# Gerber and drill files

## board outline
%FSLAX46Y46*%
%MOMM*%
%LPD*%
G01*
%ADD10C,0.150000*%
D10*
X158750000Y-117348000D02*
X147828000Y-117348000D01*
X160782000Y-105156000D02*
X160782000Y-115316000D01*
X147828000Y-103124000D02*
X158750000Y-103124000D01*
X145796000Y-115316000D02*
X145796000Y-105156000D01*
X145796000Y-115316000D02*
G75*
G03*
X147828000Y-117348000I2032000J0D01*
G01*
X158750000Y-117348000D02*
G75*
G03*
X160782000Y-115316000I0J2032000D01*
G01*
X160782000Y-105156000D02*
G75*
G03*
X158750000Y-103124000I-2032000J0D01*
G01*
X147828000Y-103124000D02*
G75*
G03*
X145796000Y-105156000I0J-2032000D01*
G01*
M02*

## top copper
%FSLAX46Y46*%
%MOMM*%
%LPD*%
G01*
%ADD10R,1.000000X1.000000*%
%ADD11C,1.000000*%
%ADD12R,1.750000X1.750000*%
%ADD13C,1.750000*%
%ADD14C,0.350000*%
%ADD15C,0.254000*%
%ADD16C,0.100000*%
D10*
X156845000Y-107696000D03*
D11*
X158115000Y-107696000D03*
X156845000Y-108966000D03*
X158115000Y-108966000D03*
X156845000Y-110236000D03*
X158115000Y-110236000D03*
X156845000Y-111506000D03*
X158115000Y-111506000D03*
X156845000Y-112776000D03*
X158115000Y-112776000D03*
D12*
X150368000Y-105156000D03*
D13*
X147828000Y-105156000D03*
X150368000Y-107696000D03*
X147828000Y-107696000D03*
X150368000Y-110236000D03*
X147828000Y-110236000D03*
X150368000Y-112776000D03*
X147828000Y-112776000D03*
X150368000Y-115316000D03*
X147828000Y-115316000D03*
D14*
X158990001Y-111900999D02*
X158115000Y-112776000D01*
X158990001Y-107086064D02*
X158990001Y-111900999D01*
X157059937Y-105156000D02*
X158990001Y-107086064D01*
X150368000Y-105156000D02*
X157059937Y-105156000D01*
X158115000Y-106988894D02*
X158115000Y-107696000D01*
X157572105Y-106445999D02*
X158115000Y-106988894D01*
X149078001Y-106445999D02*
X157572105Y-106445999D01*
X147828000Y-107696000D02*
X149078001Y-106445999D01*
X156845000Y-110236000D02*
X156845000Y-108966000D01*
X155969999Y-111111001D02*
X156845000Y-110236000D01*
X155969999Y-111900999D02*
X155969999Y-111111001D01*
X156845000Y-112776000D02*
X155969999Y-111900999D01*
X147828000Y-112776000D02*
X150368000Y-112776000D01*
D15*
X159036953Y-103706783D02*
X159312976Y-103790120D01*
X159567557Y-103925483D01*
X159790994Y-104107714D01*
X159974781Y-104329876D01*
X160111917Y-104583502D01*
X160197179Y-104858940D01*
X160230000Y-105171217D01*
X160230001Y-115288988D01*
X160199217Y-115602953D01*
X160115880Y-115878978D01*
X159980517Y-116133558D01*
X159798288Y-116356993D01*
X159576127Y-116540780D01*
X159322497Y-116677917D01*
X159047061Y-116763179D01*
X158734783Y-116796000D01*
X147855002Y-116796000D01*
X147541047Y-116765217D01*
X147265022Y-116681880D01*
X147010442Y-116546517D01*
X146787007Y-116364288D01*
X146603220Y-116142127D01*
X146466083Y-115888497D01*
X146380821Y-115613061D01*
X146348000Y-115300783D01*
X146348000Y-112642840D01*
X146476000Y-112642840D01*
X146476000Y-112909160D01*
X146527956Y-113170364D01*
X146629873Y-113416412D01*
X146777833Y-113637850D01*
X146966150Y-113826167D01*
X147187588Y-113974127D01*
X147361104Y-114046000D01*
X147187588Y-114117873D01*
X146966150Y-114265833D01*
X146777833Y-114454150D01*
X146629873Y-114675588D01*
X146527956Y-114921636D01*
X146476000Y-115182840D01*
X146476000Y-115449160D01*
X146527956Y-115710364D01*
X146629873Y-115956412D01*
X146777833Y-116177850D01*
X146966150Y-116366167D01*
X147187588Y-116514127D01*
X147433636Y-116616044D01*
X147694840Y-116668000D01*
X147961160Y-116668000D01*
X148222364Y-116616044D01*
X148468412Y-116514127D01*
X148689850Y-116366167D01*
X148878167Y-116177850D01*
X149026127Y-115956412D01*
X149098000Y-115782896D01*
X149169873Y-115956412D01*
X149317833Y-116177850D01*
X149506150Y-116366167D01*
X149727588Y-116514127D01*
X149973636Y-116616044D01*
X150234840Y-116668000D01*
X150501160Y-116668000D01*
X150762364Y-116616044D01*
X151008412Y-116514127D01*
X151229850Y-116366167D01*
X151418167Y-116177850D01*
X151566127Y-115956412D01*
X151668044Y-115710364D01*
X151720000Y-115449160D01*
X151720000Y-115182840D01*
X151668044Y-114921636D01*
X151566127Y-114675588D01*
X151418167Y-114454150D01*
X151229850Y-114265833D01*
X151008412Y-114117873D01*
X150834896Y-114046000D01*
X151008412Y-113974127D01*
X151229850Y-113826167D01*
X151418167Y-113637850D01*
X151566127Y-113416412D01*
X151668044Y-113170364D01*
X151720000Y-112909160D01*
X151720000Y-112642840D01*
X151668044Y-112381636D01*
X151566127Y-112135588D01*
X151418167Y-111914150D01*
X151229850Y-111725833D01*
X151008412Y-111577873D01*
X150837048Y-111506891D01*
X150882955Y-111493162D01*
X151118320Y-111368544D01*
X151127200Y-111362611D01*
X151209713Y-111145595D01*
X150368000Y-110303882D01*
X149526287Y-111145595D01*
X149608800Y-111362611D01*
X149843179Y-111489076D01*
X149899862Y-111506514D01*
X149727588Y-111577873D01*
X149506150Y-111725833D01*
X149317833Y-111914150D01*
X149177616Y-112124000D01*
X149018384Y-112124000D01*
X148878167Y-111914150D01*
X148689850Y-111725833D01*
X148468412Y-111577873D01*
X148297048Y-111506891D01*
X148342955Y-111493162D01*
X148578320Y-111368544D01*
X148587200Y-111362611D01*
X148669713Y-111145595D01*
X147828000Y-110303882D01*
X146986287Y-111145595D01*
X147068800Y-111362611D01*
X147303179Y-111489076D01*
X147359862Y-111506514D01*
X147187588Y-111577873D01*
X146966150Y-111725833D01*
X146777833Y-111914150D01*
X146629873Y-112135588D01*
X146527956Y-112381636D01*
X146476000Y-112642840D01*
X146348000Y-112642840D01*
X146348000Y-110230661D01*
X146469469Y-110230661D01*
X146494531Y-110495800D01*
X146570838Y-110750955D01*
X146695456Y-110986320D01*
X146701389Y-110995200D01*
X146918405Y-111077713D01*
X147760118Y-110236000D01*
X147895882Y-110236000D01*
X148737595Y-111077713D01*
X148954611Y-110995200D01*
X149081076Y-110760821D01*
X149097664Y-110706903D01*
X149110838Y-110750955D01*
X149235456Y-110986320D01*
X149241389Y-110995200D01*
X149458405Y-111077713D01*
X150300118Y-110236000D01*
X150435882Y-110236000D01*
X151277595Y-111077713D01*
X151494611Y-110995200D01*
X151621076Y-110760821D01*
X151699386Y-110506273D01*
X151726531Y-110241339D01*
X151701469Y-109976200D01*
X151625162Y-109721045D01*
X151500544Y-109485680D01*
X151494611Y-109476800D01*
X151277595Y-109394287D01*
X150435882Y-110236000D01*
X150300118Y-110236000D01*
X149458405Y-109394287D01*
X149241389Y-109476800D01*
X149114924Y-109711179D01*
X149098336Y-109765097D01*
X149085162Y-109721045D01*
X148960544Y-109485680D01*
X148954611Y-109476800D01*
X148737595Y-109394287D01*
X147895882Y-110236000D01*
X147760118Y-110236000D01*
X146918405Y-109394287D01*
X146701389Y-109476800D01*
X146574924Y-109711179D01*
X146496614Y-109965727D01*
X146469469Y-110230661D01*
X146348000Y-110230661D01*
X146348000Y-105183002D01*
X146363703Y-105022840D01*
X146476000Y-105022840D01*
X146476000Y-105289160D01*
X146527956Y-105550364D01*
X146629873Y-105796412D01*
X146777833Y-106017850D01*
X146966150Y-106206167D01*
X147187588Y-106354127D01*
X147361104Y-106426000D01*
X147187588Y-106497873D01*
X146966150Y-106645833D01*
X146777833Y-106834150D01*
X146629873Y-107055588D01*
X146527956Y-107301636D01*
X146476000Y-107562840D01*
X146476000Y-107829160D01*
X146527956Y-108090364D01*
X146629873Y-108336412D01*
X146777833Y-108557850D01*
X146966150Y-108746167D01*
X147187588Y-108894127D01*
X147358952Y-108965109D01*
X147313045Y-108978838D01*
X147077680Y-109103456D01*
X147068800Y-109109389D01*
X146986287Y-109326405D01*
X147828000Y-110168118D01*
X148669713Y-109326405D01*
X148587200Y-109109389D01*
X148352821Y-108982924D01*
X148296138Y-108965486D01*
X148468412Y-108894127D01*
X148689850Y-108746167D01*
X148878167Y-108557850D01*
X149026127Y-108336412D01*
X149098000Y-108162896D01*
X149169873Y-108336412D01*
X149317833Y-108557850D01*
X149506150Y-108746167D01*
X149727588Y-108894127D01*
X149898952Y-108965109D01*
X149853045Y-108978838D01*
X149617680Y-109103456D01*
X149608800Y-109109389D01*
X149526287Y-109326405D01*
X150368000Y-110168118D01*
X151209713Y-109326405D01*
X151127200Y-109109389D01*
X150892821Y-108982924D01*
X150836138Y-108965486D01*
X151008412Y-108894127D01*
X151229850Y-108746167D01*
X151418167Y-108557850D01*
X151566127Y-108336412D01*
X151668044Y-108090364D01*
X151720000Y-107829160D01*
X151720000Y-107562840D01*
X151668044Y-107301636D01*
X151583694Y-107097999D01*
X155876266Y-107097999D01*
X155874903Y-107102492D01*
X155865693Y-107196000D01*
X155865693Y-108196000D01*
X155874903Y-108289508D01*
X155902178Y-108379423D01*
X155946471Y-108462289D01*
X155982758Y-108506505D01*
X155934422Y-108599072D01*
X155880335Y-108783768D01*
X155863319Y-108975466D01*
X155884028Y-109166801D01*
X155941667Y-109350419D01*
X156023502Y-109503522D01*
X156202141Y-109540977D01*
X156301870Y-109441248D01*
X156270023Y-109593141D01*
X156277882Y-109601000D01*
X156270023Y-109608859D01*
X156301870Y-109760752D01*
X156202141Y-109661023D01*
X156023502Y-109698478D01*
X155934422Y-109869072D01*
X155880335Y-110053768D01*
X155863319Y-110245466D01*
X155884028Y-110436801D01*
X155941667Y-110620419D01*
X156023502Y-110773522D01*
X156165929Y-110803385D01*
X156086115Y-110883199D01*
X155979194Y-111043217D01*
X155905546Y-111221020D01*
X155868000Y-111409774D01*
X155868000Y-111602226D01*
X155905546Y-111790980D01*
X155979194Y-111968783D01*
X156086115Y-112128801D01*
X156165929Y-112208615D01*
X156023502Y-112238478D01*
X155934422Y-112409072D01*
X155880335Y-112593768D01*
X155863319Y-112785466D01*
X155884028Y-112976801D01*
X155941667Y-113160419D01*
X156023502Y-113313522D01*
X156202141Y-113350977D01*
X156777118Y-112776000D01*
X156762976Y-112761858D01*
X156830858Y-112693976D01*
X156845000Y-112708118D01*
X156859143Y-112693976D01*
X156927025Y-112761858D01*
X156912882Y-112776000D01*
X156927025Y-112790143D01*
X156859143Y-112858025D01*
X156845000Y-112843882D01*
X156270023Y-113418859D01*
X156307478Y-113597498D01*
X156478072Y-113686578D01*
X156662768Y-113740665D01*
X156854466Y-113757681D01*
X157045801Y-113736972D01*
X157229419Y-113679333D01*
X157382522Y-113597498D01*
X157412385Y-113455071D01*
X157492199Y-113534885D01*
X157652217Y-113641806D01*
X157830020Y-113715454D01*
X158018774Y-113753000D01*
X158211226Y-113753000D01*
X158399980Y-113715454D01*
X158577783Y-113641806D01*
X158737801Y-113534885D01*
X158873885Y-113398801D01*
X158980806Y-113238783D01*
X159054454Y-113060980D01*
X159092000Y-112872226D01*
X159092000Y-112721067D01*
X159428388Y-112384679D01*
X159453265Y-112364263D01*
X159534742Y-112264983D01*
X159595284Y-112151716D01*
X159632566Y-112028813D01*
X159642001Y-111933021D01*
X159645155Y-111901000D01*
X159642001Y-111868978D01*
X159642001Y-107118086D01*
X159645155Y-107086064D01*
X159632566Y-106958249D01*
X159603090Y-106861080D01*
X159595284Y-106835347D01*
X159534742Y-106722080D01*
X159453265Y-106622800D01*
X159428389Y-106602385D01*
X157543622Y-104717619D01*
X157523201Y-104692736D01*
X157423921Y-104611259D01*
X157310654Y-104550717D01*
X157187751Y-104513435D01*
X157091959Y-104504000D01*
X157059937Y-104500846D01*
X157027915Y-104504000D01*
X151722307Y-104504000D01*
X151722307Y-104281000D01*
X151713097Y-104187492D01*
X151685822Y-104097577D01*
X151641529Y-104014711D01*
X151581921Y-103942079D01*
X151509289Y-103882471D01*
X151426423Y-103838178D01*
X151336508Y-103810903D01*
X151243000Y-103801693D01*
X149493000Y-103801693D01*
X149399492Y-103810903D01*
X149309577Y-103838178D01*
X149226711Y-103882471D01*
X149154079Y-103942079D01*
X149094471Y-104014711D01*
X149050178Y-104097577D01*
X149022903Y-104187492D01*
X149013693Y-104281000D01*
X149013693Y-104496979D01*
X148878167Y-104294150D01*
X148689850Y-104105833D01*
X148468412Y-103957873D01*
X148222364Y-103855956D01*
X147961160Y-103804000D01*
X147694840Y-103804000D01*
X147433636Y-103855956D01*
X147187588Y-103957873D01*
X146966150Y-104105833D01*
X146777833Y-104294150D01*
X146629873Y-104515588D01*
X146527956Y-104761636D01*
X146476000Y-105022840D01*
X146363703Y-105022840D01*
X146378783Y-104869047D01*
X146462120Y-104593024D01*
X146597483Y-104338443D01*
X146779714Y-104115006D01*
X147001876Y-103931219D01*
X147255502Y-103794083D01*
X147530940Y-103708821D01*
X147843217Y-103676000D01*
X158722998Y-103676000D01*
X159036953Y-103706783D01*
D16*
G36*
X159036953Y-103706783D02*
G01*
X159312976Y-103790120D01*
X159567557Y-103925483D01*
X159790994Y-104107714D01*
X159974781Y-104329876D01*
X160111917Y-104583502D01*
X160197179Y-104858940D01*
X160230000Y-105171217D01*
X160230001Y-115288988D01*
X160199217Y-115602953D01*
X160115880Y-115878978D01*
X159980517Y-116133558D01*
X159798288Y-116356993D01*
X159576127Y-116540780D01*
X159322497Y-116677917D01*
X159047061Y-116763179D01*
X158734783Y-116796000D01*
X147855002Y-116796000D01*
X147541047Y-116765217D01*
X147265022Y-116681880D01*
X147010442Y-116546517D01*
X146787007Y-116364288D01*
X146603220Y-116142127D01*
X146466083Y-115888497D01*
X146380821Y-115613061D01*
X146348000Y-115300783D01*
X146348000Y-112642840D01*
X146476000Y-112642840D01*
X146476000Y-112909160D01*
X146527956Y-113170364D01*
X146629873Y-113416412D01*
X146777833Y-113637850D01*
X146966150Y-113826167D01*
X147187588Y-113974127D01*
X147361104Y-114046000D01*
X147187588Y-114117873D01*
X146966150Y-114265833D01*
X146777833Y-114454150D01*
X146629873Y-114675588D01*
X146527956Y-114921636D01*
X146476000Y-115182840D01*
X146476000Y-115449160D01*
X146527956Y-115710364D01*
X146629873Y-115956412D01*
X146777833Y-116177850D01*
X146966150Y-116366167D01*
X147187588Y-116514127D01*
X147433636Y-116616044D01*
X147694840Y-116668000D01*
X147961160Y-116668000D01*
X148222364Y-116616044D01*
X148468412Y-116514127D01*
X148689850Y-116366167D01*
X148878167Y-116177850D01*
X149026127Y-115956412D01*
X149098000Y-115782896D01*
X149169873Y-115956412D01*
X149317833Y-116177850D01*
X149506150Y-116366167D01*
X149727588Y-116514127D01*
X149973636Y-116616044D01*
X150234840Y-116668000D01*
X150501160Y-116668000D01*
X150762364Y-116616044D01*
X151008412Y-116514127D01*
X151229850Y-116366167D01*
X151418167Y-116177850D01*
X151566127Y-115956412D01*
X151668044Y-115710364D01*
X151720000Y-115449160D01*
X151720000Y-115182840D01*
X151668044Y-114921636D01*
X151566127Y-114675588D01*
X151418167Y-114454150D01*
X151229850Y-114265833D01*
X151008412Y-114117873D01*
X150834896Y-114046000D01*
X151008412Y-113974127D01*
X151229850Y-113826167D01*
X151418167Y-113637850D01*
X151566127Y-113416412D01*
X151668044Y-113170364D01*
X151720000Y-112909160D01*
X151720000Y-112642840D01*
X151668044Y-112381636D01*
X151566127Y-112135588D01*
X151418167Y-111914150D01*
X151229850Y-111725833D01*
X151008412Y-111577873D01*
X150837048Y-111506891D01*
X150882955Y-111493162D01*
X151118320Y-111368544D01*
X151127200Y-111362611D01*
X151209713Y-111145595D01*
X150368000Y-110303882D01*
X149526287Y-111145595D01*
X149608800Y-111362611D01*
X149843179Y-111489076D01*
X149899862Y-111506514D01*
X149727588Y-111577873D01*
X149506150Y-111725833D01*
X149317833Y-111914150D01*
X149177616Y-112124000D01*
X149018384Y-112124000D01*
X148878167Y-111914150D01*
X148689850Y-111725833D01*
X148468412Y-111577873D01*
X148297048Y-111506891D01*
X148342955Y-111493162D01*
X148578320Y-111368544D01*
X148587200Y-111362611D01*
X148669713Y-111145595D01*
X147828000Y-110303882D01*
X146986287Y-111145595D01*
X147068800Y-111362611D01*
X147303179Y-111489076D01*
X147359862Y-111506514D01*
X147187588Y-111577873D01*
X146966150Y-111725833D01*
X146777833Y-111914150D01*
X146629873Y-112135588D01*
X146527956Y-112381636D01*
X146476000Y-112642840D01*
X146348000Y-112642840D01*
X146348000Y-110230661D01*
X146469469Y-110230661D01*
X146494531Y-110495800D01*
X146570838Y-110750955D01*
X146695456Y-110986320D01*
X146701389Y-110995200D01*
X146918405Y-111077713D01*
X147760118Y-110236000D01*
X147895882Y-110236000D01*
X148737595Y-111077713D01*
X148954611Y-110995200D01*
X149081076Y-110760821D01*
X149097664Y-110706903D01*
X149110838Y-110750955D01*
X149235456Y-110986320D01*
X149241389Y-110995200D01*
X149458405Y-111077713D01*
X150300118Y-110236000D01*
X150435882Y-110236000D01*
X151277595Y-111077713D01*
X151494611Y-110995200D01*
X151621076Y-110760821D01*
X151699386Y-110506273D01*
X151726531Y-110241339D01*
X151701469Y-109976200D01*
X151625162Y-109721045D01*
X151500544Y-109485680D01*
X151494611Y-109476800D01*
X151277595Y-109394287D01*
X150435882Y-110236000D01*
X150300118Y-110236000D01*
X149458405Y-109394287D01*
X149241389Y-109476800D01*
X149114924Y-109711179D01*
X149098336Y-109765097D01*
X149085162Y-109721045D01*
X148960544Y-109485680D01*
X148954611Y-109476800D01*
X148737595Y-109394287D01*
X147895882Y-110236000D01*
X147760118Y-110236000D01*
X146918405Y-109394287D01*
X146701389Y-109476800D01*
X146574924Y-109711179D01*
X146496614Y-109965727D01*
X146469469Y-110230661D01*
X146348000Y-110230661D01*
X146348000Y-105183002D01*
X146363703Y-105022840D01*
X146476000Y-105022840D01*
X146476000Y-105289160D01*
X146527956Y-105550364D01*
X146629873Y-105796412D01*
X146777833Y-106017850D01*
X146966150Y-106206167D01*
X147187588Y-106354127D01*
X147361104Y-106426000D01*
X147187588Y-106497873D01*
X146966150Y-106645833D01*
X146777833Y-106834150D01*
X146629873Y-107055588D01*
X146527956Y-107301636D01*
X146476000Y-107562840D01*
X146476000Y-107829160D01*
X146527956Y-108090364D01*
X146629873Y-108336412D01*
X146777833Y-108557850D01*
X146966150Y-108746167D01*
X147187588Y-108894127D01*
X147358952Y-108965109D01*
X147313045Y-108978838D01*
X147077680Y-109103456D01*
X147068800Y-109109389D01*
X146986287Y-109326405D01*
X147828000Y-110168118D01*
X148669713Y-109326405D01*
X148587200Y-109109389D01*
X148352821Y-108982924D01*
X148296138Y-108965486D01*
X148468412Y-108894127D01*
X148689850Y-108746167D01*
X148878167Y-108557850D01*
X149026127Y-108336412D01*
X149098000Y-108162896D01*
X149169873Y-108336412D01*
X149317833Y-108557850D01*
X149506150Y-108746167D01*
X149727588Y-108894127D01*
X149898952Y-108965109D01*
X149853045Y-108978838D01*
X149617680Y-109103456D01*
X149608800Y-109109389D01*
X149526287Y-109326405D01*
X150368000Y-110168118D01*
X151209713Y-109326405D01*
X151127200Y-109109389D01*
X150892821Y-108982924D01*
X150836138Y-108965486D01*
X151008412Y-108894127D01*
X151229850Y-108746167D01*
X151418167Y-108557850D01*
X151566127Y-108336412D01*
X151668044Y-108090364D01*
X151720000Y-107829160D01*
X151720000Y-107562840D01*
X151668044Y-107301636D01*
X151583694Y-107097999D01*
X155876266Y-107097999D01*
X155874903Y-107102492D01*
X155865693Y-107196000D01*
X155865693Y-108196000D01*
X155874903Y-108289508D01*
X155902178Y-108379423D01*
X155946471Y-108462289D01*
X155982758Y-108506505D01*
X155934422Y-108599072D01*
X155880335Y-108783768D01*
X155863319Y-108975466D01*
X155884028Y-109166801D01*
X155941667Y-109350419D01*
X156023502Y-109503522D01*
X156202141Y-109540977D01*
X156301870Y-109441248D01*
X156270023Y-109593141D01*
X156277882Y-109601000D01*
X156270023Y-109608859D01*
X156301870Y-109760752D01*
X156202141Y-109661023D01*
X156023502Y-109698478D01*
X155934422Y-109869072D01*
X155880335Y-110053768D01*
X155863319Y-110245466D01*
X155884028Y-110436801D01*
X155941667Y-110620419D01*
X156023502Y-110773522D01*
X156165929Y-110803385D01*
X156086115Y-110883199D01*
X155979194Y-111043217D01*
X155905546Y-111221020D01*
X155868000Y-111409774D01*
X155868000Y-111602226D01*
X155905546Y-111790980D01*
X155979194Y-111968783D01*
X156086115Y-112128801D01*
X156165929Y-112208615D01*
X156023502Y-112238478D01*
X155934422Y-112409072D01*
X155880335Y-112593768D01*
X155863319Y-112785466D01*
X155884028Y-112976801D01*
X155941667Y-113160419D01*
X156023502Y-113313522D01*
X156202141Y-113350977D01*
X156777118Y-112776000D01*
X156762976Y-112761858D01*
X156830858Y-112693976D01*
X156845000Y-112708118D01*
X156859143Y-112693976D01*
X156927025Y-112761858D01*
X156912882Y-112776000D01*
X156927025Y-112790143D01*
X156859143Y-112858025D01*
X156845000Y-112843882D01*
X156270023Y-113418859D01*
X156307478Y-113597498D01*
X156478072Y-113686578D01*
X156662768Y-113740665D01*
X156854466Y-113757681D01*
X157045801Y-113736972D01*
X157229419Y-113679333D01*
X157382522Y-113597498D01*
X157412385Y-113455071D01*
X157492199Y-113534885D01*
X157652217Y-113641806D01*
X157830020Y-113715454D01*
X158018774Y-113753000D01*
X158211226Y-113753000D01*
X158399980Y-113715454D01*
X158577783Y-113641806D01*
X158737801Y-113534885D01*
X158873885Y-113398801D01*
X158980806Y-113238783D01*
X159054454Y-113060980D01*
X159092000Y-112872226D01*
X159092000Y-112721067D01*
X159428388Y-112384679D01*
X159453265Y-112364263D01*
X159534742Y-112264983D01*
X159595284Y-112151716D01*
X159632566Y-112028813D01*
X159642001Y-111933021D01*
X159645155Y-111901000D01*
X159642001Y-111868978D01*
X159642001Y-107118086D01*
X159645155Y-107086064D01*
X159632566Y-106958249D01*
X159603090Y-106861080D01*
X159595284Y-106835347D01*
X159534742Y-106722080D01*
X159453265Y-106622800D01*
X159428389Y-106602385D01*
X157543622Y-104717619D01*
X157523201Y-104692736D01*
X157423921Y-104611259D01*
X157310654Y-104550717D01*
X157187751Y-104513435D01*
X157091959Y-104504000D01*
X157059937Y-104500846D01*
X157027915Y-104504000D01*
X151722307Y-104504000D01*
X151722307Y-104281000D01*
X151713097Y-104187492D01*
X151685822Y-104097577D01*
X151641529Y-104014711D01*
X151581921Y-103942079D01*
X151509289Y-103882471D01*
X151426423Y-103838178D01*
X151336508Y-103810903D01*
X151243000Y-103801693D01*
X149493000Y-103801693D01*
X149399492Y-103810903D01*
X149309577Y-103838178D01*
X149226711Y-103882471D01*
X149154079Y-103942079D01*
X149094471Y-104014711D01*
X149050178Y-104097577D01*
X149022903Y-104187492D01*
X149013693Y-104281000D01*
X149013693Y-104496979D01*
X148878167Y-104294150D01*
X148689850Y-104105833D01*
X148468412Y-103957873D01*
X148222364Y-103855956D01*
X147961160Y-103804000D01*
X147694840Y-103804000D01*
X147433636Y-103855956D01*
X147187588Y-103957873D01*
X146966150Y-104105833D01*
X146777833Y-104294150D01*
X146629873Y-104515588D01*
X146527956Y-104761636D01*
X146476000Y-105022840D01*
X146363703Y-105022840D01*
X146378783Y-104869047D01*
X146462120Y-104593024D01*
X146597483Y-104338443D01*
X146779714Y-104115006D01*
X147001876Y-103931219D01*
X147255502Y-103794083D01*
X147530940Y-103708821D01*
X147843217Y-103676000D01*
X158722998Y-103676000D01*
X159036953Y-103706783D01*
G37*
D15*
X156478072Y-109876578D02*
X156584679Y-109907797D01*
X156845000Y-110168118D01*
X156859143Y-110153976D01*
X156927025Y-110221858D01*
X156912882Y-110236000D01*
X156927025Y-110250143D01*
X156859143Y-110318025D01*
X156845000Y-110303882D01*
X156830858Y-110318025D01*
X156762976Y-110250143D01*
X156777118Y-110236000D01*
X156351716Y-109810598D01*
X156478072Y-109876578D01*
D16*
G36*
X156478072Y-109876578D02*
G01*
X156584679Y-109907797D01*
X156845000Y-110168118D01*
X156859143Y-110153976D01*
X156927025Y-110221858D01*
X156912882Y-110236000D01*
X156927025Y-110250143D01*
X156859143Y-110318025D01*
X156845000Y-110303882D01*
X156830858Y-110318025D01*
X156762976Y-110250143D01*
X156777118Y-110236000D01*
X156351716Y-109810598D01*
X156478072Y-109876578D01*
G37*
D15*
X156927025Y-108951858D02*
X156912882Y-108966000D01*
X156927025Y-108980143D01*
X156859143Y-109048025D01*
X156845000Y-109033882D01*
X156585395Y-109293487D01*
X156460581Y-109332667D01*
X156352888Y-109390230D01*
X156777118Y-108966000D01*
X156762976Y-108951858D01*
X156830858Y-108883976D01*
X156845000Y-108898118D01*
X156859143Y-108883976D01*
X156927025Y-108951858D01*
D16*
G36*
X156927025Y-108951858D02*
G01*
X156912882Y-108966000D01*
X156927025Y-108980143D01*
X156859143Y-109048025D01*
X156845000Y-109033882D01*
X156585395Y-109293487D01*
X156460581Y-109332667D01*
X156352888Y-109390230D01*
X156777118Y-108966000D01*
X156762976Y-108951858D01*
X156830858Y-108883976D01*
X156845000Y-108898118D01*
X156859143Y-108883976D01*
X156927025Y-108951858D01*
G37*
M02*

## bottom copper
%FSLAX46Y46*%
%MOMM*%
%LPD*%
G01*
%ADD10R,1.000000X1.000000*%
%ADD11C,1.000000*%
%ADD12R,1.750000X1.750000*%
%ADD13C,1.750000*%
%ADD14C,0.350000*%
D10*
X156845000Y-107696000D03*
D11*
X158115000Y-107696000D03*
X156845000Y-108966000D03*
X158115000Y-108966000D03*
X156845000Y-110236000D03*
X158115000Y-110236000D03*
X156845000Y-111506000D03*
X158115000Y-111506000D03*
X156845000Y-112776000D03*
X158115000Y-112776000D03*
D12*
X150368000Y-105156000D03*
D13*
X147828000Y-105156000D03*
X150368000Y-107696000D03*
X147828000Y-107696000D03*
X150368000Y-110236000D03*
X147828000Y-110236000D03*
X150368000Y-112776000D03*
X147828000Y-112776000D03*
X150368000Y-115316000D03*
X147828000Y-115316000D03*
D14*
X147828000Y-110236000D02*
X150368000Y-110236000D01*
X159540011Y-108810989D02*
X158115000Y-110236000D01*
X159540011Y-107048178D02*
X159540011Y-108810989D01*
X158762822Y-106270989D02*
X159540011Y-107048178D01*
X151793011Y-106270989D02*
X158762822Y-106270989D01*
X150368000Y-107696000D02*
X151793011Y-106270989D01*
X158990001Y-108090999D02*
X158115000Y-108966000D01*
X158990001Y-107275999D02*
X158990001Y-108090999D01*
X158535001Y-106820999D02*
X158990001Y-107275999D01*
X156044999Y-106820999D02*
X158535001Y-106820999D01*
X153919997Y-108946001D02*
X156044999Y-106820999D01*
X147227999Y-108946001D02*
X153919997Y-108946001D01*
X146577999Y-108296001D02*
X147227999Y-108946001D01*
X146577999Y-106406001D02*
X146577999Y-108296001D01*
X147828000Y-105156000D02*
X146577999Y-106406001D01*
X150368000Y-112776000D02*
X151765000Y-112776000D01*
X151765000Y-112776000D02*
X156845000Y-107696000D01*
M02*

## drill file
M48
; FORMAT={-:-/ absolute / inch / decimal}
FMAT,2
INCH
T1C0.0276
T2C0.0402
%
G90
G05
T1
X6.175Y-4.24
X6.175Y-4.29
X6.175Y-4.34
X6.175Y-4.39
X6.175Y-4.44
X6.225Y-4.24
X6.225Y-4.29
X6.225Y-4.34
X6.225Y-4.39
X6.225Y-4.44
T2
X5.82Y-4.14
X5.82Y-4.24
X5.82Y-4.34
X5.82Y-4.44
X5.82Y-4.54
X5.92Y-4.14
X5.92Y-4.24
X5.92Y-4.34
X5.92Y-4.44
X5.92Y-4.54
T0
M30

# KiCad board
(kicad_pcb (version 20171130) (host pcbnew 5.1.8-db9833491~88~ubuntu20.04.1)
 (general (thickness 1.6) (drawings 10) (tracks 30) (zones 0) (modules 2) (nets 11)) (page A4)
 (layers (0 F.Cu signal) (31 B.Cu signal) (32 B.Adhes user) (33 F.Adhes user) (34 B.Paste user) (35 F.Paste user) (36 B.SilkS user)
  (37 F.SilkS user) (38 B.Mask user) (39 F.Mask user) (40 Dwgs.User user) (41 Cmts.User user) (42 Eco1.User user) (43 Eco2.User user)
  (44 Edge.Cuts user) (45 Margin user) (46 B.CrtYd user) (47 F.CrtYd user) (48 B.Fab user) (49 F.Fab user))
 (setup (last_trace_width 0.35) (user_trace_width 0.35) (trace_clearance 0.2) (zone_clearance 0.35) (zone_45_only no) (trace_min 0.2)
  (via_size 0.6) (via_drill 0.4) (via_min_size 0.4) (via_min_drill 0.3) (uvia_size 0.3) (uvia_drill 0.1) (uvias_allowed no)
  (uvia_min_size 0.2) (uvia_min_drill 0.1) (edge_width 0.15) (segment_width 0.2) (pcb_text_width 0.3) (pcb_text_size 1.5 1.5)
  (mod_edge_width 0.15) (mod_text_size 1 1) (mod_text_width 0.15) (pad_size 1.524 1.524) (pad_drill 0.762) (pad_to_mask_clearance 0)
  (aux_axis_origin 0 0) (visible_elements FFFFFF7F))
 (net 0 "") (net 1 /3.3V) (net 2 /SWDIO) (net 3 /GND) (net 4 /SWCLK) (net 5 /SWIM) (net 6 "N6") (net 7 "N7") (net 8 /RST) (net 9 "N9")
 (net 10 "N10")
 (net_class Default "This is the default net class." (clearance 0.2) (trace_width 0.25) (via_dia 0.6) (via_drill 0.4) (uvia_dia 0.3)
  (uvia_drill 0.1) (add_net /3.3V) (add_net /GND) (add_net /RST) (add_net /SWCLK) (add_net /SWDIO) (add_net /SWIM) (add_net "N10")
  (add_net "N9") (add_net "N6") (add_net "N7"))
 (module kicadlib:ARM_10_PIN (layer F.Cu) (at 157.48 110.236)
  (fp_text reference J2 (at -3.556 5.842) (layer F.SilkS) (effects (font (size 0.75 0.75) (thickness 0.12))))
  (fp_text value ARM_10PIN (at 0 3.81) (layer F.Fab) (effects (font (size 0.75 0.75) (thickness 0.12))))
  (pad 1 thru_hole rect (at -0.635 -2.54) (size 1 1) (drill 0.70104) (layers *.Cu *.Mask F.SilkS) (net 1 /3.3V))
  (pad 2 thru_hole circle (at 0.635 -2.54) (size 1 1) (drill 0.70104) (layers *.Cu *.Mask F.SilkS) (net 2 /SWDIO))
  (pad 3 thru_hole circle (at -0.635 -1.27) (size 1 1) (drill 0.70104) (layers *.Cu *.Mask F.SilkS) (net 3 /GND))
  (pad 4 thru_hole circle (at 0.635 -1.27) (size 1 1) (drill 0.70104) (layers *.Cu *.Mask F.SilkS) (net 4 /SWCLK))
  (pad 5 thru_hole circle (at -0.635 0) (size 1 1) (drill 0.70104) (layers *.Cu *.Mask F.SilkS) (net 3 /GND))
  (pad 6 thru_hole circle (at 0.635 0) (size 1 1) (drill 0.70104) (layers *.Cu *.Mask F.SilkS) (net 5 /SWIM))
  (pad 7 thru_hole circle (at -0.635 1.27) (size 1 1) (drill 0.70104) (layers *.Cu *.Mask F.SilkS) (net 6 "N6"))
  (pad 8 thru_hole circle (at 0.635 1.27) (size 1 1) (drill 0.70104) (layers *.Cu *.Mask F.SilkS) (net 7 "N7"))
  (pad 9 thru_hole circle (at -0.635 2.54) (size 1 1) (drill 0.70104) (layers *.Cu *.Mask F.SilkS) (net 3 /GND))
  (pad 10 thru_hole circle (at 0.635 2.54) (size 1 1) (drill 0.70104) (layers *.Cu *.Mask F.SilkS) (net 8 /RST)))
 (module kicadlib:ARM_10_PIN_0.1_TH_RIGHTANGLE (layer F.Cu) (at 150.368 105.156)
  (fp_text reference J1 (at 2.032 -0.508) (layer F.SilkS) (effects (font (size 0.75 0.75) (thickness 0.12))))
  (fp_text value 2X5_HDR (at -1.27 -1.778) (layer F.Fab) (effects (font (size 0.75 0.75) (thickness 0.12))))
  (pad 1 thru_hole rect (at 0 0) (size 1.75 1.75) (drill 1.02) (layers *.Cu *.Mask F.SilkS) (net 8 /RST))
  (pad 2 thru_hole circle (at -2.54 0) (size 1.75 1.75) (drill 1.02) (layers *.Cu *.Mask F.SilkS) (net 4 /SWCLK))
  (pad 3 thru_hole circle (at 0 2.54) (size 1.75 1.75) (drill 1.02) (layers *.Cu *.Mask F.SilkS) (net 5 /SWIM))
  (pad 4 thru_hole circle (at -2.54 2.54) (size 1.75 1.75) (drill 1.02) (layers *.Cu *.Mask F.SilkS) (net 2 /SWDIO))
  (pad 5 thru_hole circle (at 0 5.08) (size 1.75 1.75) (drill 1.02) (layers *.Cu *.Mask F.SilkS) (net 3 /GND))
  (pad 6 thru_hole circle (at -2.54 5.08) (size 1.75 1.75) (drill 1.02) (layers *.Cu *.Mask F.SilkS) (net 3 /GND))
  (pad 7 thru_hole circle (at 0 7.62) (size 1.75 1.75) (drill 1.02) (layers *.Cu *.Mask F.SilkS) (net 1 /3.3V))
  (pad 8 thru_hole circle (at -2.54 7.62) (size 1.75 1.75) (drill 1.02) (layers *.Cu *.Mask F.SilkS) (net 1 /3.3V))
  (pad 9 thru_hole circle (at 0 10.16) (size 1.75 1.75) (drill 1.02) (layers *.Cu *.Mask F.SilkS) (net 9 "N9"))
  (pad 10 thru_hole circle (at -2.54 10.16) (size 1.75 1.75) (drill 1.02) (layers *.Cu *.Mask F.SilkS) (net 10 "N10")))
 (gr_line (start 158.75 117.348) (end 147.828 117.348) (angle 90) (layer Edge.Cuts) (width 0.15))
 (gr_line (start 160.782 105.156) (end 160.782 115.316) (angle 90) (layer Edge.Cuts) (width 0.15))
 (gr_line (start 147.828 103.124) (end 158.75 103.124) (angle 90) (layer Edge.Cuts) (width 0.15))
 (gr_line (start 145.796 115.316) (end 145.796 105.156) (angle 90) (layer Edge.Cuts) (width 0.15))
 (gr_arc (start 147.828 115.316) (end 147.828 117.348) (angle 90) (layer Edge.Cuts) (width 0.15))
 (gr_arc (start 158.75 115.316) (end 160.782 115.316) (angle 90) (layer Edge.Cuts) (width 0.15))
 (gr_arc (start 158.75 105.156) (end 158.75 103.124) (angle 90) (layer Edge.Cuts) (width 0.15))
 (gr_arc (start 147.828 105.156) (end 145.796 105.156) (angle 90) (layer Edge.Cuts) (width 0.15))
 (segment (start 158.990001 111.900999) (end 158.115 112.776) (width 0.35) (layer F.Cu) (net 8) (status 20))
 (segment (start 158.990001 107.086064) (end 158.990001 111.900999) (width 0.35) (layer F.Cu) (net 8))
 (segment (start 157.059937 105.156) (end 158.990001 107.086064) (width 0.35) (layer F.Cu) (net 8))
 (segment (start 150.368 105.156) (end 157.059937 105.156) (width 0.35) (layer F.Cu) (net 8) (status 10))
 (segment (start 158.115 106.988894) (end 158.115 107.696) (width 0.35) (layer F.Cu) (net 2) (status 20))
 (segment (start 157.572105 106.445999) (end 158.115 106.988894) (width 0.35) (layer F.Cu) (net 2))
 (segment (start 149.078001 106.445999) (end 157.572105 106.445999) (width 0.35) (layer F.Cu) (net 2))
 (segment (start 147.828 107.696) (end 149.078001 106.445999) (width 0.35) (layer F.Cu) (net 2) (status 10))
 (segment (start 156.845 110.236) (end 156.845 108.966) (width 0.35) (layer F.Cu) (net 3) (status 30))
 (segment (start 147.828 110.236) (end 150.368 110.236) (width 0.35) (layer B.Cu) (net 3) (status 30))
 (segment (start 155.969999 111.111001) (end 156.845 110.236) (width 0.35) (layer F.Cu) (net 3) (status 20))
 (segment (start 155.969999 111.900999) (end 155.969999 111.111001) (width 0.35) (layer F.Cu) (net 3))
 (segment (start 156.845 112.776) (end 155.969999 111.900999) (width 0.35) (layer F.Cu) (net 3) (status 10))
 (segment (start 159.540011 108.810989) (end 158.115 110.236) (width 0.35) (layer B.Cu) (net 5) (status 20))
 (segment (start 159.540011 107.048178) (end 159.540011 108.810989) (width 0.35) (layer B.Cu) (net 5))
 (segment (start 158.762822 106.270989) (end 159.540011 107.048178) (width 0.35) (layer B.Cu) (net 5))
 (segment (start 151.793011 106.270989) (end 158.762822 106.270989) (width 0.35) (layer B.Cu) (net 5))
 (segment (start 150.368 107.696) (end 151.793011 106.270989) (width 0.35) (layer B.Cu) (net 5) (status 10))
 (segment (start 158.990001 108.090999) (end 158.115 108.966) (width 0.35) (layer B.Cu) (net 4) (status 20))
 (segment (start 158.990001 107.275999) (end 158.990001 108.090999) (width 0.35) (layer B.Cu) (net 4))
 (segment (start 158.535001 106.820999) (end 158.990001 107.275999) (width 0.35) (layer B.Cu) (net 4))
 (segment (start 156.044999 106.820999) (end 158.535001 106.820999) (width 0.35) (layer B.Cu) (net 4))
 (segment (start 153.919997 108.946001) (end 156.044999 106.820999) (width 0.35) (layer B.Cu) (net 4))
 (segment (start 147.227999 108.946001) (end 153.919997 108.946001) (width 0.35) (layer B.Cu) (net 4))
 (segment (start 146.577999 108.296001) (end 147.227999 108.946001) (width 0.35) (layer B.Cu) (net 4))
 (segment (start 146.577999 106.406001) (end 146.577999 108.296001) (width 0.35) (layer B.Cu) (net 4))
 (segment (start 147.828 105.156) (end 146.577999 106.406001) (width 0.35) (layer B.Cu) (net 4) (status 10))
 (segment (start 150.368 112.776) (end 151.765 112.776) (width 0.35) (layer B.Cu) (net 1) (status 10))
 (segment (start 151.765 112.776) (end 156.845 107.696) (width 0.35) (layer B.Cu) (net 1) (status 20))
 (segment (start 147.828 112.776) (end 150.368 112.776) (width 0.35) (layer F.Cu) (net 1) (status 30))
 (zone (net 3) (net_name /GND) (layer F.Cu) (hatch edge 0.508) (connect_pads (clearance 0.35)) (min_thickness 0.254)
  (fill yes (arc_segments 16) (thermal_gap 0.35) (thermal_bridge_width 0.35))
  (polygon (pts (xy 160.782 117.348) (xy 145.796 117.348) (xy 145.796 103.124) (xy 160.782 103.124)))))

